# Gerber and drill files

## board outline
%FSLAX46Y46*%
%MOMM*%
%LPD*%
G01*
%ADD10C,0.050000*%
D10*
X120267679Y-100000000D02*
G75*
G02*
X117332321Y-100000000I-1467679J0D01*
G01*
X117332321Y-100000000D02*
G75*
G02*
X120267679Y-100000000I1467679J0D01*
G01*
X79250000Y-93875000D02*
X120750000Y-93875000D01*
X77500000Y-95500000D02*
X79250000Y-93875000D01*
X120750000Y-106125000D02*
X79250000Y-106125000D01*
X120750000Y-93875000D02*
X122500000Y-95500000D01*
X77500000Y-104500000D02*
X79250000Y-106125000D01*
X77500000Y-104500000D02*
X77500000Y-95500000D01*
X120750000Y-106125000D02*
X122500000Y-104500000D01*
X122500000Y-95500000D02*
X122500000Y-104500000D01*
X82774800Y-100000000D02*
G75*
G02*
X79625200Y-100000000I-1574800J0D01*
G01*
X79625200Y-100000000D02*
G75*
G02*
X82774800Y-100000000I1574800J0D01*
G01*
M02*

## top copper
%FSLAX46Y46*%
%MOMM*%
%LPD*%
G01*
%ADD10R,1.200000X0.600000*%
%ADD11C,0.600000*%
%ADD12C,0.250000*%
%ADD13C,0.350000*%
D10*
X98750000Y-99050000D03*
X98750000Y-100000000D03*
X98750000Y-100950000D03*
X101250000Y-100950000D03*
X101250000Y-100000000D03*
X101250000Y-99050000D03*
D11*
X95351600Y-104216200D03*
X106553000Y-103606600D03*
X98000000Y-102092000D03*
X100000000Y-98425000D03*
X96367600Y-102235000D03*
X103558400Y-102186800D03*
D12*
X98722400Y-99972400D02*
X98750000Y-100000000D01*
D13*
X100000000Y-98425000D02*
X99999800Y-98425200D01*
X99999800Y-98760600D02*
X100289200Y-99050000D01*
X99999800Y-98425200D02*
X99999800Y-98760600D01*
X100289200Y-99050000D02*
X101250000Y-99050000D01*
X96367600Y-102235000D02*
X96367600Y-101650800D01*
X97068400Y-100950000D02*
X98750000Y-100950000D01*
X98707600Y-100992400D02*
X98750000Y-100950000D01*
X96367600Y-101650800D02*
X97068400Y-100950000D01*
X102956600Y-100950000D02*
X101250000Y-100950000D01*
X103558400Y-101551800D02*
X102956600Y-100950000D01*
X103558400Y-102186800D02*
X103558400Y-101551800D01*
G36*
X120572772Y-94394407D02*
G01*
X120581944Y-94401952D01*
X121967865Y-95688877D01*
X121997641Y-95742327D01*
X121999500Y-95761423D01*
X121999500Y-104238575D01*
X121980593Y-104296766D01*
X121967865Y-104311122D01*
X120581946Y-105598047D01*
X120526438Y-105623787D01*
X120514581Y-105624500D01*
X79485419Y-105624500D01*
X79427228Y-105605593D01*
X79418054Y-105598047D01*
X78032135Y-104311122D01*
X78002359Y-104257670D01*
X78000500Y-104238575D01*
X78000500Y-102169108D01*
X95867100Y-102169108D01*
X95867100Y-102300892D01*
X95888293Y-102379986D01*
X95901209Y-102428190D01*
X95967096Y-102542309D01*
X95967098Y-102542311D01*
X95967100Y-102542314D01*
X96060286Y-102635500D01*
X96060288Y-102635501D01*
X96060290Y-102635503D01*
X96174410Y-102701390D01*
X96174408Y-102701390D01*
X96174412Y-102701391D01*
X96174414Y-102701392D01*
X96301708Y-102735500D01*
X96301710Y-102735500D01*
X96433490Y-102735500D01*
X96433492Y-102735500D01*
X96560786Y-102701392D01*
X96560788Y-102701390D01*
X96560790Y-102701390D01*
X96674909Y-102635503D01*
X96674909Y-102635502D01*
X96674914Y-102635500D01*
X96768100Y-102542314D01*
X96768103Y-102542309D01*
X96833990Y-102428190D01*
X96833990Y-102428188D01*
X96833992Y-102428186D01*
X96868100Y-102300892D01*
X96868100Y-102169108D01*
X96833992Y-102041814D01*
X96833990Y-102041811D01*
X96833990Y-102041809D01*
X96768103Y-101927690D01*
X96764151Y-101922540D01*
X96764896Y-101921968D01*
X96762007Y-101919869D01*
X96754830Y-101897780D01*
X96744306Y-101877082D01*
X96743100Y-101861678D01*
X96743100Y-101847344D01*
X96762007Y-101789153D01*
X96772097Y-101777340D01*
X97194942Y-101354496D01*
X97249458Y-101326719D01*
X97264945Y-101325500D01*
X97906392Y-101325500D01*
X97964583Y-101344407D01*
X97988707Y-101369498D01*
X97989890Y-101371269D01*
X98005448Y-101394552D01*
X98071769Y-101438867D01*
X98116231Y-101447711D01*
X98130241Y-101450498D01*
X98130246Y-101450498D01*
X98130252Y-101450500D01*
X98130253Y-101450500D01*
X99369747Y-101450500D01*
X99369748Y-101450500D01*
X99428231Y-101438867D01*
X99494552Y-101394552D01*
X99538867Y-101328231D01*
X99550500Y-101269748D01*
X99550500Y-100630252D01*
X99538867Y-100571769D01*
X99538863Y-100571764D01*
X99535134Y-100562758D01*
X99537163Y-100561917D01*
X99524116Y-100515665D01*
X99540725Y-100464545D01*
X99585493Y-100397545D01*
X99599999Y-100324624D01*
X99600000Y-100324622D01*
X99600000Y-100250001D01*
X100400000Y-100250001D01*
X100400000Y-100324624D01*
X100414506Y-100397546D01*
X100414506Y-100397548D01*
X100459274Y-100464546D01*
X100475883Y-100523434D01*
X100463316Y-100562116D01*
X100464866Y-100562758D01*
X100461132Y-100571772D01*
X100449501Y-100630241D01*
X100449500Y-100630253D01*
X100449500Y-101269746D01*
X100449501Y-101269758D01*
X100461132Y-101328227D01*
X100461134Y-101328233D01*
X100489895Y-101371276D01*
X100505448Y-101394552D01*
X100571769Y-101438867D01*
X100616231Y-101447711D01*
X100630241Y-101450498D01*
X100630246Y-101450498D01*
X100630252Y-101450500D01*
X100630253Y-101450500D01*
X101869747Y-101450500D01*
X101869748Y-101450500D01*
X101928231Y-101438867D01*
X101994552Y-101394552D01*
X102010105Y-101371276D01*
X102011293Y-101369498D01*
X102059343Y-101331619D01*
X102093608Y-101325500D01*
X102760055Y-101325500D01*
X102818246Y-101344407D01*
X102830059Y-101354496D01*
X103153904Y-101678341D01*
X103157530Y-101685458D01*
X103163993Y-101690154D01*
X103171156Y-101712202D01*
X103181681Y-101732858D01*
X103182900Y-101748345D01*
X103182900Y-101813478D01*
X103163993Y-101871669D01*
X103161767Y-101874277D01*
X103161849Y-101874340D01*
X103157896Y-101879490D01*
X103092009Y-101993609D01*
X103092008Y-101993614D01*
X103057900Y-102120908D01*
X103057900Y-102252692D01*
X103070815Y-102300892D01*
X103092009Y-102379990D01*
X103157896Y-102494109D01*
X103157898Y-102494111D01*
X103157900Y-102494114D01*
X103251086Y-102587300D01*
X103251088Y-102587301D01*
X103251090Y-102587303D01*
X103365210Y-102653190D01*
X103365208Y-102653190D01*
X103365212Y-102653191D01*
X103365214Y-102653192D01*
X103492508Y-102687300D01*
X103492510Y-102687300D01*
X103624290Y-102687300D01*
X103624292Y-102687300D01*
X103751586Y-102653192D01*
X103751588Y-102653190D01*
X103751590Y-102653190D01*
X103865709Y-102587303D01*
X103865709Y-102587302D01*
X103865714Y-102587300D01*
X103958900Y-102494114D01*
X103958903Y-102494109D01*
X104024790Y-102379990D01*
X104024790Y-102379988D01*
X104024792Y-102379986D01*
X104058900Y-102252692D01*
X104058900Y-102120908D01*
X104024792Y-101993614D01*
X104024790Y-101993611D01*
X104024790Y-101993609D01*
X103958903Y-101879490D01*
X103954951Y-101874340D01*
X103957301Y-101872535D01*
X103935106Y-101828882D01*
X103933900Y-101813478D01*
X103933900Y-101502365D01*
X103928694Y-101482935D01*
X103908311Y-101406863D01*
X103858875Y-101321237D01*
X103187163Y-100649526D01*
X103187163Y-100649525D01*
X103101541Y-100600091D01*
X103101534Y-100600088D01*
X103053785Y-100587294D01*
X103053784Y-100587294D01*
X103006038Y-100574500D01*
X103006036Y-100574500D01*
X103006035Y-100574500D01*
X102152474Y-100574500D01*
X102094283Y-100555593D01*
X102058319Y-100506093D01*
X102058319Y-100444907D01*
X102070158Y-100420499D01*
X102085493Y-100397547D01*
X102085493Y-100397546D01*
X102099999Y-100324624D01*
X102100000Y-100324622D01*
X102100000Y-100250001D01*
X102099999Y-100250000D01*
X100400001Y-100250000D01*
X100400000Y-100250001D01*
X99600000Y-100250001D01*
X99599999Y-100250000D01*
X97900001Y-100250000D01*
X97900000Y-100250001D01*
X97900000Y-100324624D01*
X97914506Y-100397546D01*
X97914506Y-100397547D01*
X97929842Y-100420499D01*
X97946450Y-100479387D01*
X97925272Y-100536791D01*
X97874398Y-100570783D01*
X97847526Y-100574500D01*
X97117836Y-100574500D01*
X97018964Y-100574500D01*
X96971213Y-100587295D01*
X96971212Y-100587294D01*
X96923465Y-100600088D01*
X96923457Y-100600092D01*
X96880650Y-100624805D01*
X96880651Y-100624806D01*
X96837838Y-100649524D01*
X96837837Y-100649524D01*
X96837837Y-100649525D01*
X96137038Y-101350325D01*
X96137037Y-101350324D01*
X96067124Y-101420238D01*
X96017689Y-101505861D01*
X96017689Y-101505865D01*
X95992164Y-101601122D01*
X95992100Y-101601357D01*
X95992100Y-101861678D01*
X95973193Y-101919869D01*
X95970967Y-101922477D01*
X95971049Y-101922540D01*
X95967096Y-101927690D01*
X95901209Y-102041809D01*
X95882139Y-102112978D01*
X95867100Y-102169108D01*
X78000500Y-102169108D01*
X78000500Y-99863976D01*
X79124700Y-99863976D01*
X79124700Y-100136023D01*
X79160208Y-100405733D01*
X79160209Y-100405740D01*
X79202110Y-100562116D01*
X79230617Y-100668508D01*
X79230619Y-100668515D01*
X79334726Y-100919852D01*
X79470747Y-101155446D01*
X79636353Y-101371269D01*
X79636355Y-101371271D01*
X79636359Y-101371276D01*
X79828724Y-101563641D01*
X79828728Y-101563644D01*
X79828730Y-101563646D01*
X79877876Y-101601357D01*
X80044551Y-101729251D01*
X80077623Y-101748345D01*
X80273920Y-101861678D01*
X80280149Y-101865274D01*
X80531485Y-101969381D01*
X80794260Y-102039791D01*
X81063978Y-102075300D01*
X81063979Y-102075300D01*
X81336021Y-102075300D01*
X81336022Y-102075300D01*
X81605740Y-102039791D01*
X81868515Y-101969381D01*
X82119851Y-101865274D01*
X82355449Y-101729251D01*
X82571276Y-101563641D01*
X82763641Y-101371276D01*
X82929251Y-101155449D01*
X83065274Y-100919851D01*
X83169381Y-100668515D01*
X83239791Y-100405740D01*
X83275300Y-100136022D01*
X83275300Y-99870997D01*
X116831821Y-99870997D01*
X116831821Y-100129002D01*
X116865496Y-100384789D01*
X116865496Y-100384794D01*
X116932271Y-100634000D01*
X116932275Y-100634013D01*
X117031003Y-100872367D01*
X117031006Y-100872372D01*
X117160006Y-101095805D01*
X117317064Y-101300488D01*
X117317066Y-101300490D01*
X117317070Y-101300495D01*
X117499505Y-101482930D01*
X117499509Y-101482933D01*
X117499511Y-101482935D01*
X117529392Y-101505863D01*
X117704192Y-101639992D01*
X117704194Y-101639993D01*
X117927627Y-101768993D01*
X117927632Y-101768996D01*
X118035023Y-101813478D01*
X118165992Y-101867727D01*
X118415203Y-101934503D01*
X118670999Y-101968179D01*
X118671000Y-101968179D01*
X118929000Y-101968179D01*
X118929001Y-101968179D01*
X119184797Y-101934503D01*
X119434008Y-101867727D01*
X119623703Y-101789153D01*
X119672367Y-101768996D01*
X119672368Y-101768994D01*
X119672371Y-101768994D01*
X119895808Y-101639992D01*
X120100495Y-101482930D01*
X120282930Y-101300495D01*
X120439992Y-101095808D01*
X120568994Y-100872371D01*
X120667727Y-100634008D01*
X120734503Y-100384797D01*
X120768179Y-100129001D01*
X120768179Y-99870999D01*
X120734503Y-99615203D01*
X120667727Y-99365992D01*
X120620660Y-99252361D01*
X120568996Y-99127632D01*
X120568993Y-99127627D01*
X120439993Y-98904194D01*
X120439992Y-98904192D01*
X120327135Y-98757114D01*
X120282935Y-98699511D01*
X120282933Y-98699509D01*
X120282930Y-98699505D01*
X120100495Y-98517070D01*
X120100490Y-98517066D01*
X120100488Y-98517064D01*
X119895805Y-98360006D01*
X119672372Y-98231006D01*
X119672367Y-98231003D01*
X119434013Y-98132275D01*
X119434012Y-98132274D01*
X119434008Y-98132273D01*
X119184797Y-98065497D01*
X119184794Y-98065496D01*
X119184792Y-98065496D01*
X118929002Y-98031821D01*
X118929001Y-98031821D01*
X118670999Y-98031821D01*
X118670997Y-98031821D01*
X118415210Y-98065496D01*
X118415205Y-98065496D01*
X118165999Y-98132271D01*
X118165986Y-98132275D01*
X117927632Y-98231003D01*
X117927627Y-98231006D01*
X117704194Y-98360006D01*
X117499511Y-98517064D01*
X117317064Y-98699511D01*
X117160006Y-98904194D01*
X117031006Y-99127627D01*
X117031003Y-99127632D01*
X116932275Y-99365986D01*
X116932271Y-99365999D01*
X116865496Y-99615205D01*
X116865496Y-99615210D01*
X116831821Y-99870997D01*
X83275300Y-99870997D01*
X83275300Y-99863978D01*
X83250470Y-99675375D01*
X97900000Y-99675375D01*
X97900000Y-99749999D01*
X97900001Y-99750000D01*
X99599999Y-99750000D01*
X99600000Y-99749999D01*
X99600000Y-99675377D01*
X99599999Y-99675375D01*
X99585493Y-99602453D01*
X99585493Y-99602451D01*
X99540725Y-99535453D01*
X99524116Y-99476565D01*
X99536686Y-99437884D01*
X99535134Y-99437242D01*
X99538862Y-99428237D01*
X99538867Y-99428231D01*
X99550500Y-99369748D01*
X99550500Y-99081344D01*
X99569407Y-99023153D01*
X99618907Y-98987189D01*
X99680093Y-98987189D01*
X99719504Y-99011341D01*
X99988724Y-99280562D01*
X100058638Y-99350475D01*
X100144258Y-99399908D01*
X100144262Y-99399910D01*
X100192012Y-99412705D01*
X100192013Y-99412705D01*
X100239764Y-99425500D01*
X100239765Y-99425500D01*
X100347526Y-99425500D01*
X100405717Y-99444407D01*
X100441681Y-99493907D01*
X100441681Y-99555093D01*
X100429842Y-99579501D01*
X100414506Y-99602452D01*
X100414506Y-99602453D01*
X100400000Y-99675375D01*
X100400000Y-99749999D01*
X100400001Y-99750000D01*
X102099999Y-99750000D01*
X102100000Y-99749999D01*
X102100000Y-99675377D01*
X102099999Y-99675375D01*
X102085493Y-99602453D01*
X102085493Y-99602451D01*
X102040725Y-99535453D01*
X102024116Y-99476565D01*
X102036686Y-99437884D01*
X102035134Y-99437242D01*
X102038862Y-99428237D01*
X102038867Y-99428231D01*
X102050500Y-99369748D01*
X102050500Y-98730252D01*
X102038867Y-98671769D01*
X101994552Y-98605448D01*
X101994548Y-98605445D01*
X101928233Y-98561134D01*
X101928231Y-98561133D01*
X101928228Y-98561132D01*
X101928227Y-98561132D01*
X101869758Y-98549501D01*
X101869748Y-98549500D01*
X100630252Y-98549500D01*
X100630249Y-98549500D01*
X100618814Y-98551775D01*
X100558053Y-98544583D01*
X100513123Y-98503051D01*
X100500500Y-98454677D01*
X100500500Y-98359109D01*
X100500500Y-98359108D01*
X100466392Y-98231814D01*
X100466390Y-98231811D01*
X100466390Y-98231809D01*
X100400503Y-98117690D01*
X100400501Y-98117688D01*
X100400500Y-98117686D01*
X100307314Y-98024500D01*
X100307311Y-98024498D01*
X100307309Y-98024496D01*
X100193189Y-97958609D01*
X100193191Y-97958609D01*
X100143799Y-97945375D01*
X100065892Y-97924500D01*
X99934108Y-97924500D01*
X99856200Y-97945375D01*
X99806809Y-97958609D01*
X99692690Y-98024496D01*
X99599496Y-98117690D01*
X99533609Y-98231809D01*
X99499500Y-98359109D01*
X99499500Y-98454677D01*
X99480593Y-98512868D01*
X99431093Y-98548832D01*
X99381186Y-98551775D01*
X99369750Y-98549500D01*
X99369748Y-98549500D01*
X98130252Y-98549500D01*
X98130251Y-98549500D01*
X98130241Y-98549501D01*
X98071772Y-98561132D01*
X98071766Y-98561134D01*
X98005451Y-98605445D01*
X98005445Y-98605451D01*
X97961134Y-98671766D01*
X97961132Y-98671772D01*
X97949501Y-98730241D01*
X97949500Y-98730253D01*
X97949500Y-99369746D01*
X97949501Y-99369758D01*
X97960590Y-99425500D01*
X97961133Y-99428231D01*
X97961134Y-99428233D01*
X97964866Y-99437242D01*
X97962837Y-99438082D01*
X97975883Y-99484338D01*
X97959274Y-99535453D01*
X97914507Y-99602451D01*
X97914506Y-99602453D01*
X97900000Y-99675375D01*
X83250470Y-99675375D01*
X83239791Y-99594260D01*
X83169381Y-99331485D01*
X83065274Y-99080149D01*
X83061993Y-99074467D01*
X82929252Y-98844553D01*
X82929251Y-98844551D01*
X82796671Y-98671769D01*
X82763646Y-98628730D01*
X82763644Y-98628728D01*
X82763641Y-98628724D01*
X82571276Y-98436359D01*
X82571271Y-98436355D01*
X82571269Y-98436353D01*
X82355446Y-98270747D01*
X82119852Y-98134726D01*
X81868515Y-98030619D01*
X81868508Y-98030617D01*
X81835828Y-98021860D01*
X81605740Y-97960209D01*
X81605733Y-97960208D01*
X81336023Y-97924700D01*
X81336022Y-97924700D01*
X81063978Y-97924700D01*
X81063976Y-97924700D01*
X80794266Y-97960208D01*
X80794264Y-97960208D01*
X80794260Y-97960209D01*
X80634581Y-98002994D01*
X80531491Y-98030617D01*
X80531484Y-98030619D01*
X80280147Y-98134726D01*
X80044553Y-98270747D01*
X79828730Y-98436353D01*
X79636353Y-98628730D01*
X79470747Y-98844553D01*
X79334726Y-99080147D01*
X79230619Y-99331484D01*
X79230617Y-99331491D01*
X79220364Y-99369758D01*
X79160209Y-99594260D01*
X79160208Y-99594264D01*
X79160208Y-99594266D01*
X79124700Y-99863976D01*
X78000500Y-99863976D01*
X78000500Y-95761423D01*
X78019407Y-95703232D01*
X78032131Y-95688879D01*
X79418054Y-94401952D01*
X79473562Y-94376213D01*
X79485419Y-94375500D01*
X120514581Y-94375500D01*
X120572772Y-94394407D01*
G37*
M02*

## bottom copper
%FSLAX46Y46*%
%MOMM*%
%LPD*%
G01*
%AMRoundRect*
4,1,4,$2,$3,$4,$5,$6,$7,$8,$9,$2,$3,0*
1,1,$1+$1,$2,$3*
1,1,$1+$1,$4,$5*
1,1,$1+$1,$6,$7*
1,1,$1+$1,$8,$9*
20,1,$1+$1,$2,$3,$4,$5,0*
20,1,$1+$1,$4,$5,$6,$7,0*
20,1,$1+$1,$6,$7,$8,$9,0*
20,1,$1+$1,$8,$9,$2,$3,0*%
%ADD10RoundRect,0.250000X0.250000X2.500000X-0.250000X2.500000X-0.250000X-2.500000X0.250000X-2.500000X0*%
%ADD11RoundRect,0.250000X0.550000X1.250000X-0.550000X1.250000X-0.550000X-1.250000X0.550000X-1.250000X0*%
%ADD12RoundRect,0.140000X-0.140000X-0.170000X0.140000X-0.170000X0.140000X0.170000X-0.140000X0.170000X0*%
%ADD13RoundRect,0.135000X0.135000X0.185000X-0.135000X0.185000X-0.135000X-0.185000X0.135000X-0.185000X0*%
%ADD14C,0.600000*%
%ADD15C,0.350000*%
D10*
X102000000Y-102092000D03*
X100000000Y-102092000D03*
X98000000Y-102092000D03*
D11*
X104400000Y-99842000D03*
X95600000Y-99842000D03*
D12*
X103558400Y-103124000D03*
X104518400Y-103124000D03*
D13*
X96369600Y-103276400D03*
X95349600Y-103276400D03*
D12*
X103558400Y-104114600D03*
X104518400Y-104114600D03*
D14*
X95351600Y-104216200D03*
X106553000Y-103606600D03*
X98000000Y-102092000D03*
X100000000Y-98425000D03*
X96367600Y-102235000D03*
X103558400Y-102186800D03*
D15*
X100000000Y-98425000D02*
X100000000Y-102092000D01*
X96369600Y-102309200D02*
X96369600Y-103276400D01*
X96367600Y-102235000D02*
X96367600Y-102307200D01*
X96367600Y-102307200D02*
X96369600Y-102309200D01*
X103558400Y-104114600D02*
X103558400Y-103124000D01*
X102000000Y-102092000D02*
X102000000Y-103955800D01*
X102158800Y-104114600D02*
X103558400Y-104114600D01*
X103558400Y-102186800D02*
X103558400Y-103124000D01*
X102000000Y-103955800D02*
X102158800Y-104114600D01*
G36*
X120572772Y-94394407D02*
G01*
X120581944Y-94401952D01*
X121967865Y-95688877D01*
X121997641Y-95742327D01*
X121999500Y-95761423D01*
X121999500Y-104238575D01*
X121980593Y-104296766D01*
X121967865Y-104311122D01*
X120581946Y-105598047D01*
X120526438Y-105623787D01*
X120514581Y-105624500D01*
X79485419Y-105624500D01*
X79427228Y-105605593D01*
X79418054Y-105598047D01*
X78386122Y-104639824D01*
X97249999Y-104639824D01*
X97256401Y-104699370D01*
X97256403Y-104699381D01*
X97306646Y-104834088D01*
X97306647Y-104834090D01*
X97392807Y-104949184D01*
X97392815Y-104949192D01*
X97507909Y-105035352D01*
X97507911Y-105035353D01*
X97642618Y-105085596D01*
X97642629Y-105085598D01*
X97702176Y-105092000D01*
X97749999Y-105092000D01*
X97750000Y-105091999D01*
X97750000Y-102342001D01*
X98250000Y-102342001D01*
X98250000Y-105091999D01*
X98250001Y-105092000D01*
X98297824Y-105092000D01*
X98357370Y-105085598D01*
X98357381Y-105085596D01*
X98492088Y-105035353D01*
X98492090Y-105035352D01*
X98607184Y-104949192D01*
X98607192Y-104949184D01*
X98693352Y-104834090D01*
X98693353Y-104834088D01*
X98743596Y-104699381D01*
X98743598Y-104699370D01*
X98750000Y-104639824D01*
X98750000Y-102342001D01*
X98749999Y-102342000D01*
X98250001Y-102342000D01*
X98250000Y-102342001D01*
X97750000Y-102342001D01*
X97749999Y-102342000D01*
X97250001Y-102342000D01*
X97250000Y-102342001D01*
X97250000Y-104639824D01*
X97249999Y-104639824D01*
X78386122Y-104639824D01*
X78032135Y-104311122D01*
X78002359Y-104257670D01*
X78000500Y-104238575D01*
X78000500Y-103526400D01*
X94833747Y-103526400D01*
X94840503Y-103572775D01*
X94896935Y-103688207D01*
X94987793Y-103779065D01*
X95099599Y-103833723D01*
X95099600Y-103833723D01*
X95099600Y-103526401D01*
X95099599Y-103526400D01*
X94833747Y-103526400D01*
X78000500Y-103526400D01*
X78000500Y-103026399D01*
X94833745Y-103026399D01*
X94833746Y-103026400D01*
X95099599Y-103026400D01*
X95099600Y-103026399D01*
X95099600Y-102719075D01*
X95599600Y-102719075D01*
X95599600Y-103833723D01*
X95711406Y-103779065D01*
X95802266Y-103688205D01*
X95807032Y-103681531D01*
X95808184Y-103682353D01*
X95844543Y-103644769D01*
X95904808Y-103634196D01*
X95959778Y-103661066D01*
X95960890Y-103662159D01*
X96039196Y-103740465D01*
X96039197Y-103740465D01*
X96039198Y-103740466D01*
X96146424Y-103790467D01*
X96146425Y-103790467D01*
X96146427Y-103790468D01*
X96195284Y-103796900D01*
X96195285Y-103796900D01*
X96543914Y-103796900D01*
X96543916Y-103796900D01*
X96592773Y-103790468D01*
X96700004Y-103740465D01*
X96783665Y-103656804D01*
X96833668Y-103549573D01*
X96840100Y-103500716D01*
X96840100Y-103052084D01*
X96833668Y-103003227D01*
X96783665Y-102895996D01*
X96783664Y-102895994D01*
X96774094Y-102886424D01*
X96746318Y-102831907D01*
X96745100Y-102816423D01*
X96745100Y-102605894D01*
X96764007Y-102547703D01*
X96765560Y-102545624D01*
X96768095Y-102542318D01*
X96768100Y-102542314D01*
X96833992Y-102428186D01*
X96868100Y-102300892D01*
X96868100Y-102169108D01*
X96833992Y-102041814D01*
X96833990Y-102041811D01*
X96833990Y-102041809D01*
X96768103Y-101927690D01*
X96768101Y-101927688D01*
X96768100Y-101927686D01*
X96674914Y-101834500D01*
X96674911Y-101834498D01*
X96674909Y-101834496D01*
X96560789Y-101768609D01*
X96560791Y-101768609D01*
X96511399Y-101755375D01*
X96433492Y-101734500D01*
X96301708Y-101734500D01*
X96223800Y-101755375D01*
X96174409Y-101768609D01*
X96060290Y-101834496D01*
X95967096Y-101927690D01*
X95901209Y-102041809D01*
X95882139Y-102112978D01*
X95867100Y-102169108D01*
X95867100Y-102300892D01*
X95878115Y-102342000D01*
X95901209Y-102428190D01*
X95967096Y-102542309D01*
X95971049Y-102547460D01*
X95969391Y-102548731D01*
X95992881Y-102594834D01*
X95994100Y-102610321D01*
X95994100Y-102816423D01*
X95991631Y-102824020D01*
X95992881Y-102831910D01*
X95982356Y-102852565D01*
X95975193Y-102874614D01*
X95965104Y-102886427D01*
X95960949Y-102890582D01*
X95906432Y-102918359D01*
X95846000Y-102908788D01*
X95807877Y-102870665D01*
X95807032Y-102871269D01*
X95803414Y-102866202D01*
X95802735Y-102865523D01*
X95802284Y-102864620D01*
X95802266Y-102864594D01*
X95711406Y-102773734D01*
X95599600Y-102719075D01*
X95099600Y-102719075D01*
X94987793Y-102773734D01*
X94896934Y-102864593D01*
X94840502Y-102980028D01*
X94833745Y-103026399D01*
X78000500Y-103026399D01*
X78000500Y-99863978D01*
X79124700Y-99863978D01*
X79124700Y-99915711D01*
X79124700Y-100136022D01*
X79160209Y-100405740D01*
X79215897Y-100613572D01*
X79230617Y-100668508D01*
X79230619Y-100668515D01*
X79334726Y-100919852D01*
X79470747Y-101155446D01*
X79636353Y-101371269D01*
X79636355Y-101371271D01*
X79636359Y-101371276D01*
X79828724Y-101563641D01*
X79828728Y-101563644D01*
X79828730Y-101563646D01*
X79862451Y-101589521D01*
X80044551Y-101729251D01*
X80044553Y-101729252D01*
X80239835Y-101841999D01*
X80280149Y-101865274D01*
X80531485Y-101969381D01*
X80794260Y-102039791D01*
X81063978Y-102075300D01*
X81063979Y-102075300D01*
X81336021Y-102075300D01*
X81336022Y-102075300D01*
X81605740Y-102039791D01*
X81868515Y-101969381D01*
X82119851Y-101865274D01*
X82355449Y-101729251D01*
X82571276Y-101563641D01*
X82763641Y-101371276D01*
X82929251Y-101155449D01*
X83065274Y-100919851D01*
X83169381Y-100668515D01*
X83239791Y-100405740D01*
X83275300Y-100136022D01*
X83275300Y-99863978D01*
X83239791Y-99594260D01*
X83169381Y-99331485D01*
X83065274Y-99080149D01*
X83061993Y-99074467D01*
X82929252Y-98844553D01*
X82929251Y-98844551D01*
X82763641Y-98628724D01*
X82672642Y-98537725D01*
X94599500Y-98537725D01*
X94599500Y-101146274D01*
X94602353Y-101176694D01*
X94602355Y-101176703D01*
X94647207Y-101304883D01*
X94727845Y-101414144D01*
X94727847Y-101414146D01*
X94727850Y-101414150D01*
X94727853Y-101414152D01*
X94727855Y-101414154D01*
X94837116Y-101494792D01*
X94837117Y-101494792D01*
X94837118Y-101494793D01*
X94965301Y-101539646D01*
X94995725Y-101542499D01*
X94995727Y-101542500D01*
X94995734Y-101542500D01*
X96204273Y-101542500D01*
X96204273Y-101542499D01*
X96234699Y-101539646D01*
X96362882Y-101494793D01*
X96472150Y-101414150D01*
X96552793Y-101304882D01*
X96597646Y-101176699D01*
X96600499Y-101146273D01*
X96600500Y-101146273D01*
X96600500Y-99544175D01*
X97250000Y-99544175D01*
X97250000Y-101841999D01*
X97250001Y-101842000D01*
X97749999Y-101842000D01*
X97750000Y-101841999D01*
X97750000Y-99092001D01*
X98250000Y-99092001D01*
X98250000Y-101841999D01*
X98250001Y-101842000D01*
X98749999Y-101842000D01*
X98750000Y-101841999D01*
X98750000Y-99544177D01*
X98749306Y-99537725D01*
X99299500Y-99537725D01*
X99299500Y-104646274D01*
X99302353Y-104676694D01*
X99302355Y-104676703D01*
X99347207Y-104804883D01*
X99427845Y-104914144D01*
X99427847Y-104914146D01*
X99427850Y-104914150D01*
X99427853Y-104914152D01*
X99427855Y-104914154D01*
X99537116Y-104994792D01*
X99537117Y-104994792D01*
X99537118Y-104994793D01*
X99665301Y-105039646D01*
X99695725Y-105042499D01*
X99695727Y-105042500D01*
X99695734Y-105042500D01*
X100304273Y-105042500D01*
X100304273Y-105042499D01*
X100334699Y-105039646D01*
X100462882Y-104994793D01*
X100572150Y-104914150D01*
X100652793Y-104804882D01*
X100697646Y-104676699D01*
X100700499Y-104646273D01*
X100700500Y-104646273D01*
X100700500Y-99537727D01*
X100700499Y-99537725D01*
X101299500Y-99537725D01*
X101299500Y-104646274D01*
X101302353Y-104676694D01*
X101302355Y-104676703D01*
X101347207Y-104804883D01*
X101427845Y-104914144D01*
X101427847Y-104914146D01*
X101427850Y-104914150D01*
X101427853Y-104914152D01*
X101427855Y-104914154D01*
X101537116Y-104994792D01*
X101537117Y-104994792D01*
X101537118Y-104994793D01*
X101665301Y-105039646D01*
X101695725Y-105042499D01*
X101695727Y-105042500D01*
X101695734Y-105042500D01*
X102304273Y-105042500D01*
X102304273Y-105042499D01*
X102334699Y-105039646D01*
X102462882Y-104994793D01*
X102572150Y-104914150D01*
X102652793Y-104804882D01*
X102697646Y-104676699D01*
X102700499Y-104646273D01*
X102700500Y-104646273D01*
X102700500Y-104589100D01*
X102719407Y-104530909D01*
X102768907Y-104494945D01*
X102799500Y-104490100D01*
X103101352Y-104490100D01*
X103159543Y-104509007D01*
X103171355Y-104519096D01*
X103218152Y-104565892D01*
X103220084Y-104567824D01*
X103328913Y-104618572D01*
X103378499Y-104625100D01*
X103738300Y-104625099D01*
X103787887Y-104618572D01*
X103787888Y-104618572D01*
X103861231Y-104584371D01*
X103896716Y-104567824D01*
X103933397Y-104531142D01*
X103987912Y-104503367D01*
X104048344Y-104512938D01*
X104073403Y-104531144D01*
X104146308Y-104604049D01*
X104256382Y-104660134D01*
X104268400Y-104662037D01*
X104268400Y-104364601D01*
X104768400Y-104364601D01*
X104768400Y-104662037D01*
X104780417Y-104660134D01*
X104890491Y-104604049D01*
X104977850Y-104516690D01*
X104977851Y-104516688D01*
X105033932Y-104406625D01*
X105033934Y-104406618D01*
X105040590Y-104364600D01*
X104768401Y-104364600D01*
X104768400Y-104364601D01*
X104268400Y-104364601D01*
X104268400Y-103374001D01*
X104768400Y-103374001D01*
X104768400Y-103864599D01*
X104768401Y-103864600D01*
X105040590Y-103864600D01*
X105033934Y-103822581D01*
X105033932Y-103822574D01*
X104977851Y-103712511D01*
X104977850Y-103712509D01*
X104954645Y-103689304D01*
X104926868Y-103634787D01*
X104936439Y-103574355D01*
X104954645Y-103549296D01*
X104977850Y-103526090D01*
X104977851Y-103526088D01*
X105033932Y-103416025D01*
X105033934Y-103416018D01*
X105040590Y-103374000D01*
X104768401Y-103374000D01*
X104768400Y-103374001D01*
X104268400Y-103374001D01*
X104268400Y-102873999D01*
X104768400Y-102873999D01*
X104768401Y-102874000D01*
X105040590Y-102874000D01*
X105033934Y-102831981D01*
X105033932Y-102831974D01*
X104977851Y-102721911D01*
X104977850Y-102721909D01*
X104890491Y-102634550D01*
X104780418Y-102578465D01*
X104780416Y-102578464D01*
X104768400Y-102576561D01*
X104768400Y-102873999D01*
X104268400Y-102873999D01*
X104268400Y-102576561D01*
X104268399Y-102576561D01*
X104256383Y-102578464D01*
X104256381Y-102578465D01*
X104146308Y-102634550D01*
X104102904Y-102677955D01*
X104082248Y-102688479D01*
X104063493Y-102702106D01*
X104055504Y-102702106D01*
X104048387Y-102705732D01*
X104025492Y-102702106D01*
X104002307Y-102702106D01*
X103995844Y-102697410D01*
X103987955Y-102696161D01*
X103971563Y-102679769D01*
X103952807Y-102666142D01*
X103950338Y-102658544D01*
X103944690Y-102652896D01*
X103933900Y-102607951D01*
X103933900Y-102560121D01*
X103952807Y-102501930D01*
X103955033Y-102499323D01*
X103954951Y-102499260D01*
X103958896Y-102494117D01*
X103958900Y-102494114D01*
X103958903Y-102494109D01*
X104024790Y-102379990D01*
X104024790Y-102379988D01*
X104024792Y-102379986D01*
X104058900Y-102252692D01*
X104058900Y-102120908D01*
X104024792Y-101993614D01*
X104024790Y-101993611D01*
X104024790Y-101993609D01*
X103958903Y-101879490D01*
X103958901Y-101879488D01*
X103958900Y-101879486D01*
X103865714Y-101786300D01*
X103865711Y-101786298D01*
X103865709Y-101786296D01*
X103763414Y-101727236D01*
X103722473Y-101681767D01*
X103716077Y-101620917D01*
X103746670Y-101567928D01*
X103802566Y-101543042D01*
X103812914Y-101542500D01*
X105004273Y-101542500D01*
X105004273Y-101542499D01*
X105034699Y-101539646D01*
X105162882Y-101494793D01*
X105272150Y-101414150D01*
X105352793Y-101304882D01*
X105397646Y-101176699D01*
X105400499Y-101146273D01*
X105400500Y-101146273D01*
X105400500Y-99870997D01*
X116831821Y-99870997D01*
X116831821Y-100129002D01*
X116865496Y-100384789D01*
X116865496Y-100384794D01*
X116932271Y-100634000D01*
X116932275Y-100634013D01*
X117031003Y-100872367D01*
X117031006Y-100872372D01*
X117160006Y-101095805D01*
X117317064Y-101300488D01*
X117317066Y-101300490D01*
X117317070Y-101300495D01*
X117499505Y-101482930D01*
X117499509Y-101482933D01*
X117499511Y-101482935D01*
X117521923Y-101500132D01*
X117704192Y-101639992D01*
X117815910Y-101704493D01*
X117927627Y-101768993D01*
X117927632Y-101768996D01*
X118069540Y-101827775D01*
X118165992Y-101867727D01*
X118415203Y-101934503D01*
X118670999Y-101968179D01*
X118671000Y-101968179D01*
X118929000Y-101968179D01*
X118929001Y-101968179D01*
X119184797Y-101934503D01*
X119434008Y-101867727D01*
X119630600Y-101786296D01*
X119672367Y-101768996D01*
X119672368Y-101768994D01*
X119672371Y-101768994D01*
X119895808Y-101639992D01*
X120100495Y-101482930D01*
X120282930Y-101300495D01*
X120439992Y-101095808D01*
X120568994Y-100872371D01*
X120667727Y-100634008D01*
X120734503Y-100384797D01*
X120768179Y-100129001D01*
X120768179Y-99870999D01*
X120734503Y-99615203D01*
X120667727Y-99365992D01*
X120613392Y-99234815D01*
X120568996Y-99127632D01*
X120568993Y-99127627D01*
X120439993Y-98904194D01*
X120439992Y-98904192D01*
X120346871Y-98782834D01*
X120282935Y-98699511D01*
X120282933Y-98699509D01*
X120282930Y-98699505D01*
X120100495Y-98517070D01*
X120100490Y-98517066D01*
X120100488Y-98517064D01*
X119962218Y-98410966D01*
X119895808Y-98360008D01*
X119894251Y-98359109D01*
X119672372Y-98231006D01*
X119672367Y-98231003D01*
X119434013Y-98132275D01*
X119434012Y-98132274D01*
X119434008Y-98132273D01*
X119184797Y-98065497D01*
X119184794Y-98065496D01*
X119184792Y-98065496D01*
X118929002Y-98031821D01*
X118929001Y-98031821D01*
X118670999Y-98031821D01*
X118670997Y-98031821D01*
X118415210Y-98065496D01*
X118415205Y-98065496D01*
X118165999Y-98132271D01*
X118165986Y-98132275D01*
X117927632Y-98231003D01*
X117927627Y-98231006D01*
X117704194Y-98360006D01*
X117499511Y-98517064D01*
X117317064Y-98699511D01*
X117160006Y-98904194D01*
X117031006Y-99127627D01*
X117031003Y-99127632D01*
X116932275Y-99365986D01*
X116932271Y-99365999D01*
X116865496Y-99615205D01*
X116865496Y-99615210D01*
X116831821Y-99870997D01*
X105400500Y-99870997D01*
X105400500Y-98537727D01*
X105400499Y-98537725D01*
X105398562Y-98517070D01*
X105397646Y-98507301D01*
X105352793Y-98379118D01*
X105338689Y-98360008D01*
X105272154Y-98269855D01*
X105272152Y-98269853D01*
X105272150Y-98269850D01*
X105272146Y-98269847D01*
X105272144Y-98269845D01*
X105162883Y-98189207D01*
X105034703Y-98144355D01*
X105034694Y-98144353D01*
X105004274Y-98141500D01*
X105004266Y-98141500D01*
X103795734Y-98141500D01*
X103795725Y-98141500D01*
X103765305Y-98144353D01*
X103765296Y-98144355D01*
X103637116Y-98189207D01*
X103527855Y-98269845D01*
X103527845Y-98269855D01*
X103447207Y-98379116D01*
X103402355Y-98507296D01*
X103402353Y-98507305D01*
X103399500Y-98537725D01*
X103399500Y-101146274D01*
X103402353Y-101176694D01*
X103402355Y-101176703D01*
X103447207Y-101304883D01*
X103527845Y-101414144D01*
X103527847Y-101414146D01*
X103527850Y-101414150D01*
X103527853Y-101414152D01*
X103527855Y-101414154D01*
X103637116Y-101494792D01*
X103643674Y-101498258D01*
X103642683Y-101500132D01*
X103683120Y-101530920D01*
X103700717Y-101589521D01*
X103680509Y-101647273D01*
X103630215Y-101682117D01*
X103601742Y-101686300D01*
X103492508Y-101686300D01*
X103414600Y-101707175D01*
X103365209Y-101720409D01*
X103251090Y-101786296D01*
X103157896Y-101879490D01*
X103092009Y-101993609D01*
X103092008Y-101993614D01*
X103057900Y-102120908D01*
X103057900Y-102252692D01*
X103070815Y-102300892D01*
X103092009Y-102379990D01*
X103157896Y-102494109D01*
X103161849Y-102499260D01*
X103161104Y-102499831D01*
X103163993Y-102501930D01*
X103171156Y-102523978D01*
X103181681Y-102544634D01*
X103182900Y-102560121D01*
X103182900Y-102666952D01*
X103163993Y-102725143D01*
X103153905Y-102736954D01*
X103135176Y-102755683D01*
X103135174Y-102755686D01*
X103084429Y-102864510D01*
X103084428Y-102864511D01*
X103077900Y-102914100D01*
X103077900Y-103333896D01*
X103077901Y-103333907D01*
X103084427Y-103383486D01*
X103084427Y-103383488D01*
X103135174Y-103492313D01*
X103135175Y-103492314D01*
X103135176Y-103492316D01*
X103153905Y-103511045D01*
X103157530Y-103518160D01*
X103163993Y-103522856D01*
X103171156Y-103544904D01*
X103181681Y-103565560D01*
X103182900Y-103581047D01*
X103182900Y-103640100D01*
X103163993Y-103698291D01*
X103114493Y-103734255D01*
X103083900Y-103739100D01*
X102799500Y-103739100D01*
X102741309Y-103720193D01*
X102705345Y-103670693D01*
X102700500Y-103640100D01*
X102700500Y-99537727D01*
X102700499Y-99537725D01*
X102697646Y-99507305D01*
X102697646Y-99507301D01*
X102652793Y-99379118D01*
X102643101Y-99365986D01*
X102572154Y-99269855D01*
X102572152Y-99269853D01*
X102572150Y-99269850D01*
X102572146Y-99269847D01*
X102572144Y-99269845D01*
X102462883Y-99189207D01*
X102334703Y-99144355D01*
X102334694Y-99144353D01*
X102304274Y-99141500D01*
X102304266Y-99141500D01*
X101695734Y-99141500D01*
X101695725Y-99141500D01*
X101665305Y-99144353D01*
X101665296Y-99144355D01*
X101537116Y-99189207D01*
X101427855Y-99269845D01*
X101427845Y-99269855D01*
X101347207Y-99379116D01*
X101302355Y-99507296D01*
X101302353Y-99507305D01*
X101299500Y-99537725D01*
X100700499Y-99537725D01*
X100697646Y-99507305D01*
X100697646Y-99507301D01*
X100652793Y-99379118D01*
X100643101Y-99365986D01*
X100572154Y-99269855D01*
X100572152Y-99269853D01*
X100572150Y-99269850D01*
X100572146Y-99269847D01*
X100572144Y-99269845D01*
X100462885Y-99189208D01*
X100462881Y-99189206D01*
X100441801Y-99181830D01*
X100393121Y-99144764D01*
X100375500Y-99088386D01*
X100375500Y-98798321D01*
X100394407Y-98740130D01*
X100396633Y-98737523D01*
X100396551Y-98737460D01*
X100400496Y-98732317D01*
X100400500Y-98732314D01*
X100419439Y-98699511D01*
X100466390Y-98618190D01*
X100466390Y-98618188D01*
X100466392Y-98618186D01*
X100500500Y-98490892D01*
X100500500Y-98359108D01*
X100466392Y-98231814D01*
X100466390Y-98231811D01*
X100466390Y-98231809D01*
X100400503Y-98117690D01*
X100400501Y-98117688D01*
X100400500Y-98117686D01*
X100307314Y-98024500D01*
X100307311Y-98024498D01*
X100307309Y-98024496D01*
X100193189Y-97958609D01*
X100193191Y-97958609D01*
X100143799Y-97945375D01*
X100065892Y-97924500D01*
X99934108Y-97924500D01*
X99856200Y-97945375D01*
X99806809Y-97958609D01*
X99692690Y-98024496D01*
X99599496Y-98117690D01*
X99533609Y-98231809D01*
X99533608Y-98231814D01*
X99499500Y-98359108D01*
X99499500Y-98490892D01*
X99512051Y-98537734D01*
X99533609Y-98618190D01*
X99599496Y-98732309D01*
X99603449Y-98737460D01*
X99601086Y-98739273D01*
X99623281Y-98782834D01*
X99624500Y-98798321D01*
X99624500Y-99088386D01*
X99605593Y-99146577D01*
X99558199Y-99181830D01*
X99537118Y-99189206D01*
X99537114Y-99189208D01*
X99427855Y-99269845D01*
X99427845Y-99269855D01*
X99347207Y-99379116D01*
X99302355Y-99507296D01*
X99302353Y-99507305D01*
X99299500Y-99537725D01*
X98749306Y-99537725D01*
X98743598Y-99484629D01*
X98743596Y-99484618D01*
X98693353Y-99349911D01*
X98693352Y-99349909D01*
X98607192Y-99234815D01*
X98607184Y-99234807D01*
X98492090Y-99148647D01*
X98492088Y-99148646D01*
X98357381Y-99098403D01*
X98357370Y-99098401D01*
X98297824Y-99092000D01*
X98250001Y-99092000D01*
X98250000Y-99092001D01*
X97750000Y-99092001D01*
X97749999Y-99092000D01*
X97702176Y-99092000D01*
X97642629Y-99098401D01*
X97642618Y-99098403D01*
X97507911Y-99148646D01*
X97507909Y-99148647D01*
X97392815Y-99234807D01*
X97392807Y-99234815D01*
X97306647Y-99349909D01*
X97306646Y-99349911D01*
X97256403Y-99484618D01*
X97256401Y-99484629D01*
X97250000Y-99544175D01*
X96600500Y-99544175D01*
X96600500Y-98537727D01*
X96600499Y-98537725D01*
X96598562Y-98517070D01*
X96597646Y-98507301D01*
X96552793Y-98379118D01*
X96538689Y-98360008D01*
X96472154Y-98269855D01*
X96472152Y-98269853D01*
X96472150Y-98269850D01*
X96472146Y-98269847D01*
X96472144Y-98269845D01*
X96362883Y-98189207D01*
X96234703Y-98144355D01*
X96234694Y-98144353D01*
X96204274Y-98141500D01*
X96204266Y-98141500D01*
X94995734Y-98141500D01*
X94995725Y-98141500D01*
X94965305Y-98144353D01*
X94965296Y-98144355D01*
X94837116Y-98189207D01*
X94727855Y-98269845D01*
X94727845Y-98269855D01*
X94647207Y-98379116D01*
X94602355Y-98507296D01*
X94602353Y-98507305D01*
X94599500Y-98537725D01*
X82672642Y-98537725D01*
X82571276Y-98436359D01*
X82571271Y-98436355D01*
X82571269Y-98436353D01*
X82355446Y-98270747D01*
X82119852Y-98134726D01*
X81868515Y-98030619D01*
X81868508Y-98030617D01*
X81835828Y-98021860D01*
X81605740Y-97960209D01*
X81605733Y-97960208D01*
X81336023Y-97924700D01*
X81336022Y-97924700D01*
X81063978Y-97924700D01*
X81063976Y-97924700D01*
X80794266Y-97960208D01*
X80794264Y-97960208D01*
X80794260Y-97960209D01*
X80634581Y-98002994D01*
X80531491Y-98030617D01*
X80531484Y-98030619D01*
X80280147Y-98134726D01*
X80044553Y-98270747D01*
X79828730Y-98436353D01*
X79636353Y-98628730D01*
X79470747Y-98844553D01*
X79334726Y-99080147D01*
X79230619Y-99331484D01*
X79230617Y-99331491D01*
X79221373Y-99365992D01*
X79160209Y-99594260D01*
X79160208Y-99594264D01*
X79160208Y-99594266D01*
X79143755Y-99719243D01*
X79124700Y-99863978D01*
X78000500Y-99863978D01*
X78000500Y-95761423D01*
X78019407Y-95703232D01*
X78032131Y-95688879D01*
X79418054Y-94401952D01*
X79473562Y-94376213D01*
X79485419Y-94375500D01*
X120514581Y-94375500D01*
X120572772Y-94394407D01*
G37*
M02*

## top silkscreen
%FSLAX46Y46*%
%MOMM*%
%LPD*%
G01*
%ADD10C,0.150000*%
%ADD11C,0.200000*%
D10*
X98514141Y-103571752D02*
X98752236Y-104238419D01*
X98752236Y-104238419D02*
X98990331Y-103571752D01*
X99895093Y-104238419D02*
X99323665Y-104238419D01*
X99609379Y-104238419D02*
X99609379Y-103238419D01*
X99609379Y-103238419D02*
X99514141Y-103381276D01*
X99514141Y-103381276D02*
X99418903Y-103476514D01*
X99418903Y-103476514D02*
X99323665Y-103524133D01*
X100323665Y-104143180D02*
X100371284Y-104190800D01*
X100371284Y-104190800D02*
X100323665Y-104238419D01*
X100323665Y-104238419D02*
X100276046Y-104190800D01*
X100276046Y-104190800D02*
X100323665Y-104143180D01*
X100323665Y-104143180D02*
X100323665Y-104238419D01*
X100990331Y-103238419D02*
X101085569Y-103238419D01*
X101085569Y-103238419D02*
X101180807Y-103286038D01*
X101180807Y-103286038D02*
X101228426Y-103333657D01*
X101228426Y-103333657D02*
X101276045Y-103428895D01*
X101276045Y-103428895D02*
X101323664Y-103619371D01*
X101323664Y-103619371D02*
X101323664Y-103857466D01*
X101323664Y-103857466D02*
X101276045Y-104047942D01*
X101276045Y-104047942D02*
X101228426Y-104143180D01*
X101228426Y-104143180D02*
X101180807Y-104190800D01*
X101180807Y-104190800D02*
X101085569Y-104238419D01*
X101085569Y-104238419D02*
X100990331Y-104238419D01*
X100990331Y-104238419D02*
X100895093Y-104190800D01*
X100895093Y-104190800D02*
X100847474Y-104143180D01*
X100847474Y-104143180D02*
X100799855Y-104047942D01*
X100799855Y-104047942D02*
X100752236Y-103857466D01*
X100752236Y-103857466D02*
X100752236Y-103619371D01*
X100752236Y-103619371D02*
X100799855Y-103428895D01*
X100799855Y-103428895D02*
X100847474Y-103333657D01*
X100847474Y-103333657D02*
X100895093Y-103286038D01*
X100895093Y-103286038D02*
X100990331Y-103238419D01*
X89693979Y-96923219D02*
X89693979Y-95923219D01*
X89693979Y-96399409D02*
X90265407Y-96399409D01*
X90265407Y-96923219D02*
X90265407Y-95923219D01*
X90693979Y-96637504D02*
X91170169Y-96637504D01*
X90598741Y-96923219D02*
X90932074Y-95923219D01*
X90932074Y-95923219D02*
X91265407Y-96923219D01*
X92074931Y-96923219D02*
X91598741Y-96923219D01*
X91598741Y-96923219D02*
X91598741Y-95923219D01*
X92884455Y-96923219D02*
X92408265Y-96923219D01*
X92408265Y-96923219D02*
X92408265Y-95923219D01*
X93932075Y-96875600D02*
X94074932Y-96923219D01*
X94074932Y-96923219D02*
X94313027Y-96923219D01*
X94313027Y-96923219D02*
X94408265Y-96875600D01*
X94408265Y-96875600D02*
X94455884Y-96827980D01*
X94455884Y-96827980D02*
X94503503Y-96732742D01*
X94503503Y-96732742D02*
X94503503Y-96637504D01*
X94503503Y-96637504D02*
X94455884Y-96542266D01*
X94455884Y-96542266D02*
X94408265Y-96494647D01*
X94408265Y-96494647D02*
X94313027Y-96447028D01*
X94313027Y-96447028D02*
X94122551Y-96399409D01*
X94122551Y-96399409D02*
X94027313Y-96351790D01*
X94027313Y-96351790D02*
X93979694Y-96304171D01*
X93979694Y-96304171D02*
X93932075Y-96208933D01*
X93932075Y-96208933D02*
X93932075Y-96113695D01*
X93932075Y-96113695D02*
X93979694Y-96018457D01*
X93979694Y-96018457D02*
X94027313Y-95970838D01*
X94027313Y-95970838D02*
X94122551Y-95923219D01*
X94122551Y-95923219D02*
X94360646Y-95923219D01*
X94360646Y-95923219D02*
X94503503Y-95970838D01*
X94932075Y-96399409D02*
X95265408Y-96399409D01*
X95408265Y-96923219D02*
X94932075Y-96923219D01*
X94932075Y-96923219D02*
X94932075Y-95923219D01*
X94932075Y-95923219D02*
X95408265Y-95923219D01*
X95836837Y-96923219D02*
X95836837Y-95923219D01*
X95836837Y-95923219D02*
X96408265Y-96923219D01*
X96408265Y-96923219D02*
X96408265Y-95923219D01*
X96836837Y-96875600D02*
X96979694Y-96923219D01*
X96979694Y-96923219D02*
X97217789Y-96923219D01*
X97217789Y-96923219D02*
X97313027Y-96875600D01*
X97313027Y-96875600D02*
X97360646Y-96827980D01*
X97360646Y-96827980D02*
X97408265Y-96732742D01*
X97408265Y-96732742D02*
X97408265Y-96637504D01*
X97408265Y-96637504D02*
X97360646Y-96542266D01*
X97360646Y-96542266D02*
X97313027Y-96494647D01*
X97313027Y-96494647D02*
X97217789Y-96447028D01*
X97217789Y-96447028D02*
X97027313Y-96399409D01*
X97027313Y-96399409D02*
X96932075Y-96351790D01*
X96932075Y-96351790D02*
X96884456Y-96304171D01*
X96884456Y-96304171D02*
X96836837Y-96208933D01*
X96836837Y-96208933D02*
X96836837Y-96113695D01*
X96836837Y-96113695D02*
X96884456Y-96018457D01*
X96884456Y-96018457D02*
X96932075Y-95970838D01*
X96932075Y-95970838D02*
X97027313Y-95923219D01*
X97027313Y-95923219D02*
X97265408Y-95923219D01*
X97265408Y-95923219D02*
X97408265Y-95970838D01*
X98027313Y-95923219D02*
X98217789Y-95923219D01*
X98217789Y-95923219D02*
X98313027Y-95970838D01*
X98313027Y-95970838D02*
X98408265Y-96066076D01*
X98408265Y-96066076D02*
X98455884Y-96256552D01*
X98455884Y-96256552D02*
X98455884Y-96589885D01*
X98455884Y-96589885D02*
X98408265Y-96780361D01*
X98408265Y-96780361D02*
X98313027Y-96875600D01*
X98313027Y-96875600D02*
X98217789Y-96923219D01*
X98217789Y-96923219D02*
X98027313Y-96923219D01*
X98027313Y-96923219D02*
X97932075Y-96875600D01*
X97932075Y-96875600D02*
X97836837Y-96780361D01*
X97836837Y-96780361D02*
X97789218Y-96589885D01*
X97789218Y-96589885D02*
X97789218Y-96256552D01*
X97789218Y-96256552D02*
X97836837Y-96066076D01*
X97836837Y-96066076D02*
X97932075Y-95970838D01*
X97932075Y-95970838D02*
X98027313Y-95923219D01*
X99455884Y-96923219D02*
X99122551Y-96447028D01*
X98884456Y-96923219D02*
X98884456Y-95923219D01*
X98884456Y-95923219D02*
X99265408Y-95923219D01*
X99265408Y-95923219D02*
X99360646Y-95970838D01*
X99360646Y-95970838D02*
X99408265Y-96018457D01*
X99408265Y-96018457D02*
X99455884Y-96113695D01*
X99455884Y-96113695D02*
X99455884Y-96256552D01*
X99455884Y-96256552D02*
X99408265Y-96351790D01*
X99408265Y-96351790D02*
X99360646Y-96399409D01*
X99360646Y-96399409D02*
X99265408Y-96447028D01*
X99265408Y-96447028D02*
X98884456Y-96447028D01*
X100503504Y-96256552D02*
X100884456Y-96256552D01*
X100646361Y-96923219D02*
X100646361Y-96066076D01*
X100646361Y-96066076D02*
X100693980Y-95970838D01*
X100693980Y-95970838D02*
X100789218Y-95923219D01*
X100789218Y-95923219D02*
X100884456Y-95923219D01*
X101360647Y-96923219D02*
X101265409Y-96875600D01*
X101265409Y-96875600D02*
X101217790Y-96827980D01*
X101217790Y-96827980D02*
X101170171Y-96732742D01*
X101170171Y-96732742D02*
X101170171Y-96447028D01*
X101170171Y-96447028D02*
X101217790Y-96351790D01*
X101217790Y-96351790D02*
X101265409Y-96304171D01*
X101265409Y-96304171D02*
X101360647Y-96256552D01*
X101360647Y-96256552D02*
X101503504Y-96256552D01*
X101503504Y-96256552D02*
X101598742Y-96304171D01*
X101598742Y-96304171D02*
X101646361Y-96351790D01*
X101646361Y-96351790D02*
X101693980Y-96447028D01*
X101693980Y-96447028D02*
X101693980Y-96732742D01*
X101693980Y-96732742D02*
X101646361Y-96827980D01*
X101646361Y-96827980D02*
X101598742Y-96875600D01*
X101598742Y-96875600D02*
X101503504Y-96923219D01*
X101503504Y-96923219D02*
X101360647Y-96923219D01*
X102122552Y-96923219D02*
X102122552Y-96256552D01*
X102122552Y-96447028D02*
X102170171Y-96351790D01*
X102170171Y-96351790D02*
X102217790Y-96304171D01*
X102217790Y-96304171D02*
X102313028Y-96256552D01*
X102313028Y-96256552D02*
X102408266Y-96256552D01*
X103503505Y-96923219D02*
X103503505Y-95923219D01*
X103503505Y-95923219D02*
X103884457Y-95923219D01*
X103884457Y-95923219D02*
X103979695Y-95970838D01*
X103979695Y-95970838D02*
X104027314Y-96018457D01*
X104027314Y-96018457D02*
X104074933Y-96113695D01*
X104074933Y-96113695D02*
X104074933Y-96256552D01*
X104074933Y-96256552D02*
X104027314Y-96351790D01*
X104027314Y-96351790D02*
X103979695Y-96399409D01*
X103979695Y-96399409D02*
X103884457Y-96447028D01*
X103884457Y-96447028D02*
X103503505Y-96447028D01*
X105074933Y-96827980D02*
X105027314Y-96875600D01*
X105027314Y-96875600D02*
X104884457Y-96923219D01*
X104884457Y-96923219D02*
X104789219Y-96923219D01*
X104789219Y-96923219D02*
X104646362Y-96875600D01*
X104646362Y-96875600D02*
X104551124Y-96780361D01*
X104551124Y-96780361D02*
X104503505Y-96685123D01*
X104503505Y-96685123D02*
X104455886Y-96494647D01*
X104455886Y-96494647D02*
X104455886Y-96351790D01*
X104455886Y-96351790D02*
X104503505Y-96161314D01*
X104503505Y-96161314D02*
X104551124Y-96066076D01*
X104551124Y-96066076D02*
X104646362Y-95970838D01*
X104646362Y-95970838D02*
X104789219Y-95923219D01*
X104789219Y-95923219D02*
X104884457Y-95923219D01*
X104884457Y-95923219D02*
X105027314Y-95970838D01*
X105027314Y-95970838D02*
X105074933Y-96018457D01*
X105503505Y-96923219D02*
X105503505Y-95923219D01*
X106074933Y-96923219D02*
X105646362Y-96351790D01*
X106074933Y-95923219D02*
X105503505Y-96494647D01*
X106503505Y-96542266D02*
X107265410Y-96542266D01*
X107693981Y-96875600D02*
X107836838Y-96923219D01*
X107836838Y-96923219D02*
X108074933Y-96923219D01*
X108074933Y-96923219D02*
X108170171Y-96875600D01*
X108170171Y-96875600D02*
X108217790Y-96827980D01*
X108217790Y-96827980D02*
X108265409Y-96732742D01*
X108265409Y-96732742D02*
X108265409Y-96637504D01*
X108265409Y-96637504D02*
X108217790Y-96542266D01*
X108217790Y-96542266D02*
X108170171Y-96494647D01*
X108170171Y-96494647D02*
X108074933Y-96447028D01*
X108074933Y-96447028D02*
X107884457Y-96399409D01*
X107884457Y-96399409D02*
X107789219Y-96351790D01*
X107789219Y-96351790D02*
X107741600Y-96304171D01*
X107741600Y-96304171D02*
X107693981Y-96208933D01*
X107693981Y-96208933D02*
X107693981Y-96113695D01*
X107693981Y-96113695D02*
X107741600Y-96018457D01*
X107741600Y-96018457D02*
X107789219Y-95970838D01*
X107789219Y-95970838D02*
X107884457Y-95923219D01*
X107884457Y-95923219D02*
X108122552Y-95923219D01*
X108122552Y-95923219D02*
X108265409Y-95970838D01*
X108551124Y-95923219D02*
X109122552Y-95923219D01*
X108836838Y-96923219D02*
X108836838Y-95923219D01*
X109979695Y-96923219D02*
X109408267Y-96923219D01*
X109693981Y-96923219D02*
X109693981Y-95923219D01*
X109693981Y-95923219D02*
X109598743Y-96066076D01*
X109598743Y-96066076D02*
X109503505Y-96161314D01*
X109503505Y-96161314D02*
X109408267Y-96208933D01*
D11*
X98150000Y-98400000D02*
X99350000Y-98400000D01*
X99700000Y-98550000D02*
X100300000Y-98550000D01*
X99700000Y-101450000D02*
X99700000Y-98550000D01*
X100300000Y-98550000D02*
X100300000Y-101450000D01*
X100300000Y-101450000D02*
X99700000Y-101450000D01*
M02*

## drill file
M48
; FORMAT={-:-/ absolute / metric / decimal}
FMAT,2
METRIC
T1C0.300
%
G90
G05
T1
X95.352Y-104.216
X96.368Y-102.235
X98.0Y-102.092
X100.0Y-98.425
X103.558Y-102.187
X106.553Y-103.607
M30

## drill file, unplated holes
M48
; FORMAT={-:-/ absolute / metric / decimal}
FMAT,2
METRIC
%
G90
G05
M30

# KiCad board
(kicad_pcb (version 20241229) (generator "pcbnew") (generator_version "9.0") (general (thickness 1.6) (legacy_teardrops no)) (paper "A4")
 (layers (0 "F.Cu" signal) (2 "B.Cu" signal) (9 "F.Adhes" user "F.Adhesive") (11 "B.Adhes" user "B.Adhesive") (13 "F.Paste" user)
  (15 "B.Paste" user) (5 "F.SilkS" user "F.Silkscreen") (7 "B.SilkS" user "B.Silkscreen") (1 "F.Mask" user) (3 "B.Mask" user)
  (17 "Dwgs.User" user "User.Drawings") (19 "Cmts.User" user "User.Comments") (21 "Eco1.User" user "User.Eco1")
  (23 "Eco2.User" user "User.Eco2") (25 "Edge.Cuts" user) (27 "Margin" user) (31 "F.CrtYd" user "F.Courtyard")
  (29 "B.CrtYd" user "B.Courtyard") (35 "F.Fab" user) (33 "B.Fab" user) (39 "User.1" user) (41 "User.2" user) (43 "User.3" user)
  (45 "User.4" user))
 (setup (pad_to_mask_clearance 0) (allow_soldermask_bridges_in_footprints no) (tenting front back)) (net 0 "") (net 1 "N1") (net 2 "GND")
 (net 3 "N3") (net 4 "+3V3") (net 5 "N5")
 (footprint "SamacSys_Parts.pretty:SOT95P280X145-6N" (layer "F.Cu") (at 100 100)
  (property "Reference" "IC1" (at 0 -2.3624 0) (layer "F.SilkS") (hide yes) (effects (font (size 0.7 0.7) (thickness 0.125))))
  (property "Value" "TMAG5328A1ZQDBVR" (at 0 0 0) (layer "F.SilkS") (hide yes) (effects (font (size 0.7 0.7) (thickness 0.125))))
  (fp_line (start -1.85 -1.6) (end -0.65 -1.6) (stroke (width 0.2) (type solid)) (layer "F.SilkS"))
  (fp_line (start -0.3 -1.45) (end 0.3 -1.45) (stroke (width 0.2) (type solid)) (layer "F.SilkS"))
  (fp_line (start -0.3 1.45) (end -0.3 -1.45) (stroke (width 0.2) (type solid)) (layer "F.SilkS"))
  (fp_line (start 0.3 -1.45) (end 0.3 1.45) (stroke (width 0.2) (type solid)) (layer "F.SilkS"))
  (fp_line (start 0.3 1.45) (end -0.3 1.45) (stroke (width 0.2) (type solid)) (layer "F.SilkS"))
  (pad "1" smd rect (at -1.25 -0.95 90) (size 0.6 1.2) (layers "F.Cu" "F.Mask" "F.Paste") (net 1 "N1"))
  (pad "2" smd rect (at -1.25 0 90) (size 0.6 1.2) (layers "F.Cu" "F.Mask" "F.Paste") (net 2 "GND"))
  (pad "3" smd rect (at -1.25 0.95 90) (size 0.6 1.2) (layers "F.Cu" "F.Mask" "F.Paste") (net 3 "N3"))
  (pad "4" smd rect (at 1.25 0.95 90) (size 0.6 1.2) (layers "F.Cu" "F.Mask" "F.Paste") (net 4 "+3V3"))
  (pad "5" smd rect (at 1.25 0 90) (size 0.6 1.2) (layers "F.Cu" "F.Mask" "F.Paste") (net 2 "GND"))
  (pad "6" smd rect (at 1.25 -0.95 90) (size 0.6 1.2) (layers "F.Cu" "F.Mask" "F.Paste") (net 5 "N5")))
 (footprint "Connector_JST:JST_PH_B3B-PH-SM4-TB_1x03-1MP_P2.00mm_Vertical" (layer "B.Cu") (at 100 101.592 180)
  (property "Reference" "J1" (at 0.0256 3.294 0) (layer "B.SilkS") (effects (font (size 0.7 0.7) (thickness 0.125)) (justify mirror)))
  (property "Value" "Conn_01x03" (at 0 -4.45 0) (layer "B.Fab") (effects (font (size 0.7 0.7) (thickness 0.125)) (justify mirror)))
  (pad "1" smd roundrect (at -2 -0.5 180) (size 1 5.5) (layers "B.Cu" "B.Mask" "B.Paste") (roundrect_rratio 0.25) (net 4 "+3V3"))
  (pad "2" smd roundrect (at 0 -0.5 180) (size 1 5.5) (layers "B.Cu" "B.Mask" "B.Paste") (roundrect_rratio 0.25) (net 5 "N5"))
  (pad "3" smd roundrect (at 2 -0.5 180) (size 1 5.5) (layers "B.Cu" "B.Mask" "B.Paste") (roundrect_rratio 0.25) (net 2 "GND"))
  (pad "MP" smd roundrect (at -4.4 1.75 180) (size 1.6 3) (layers "B.Cu" "B.Mask" "B.Paste") (roundrect_rratio 0.15625))
  (pad "MP" smd roundrect (at 4.4 1.75 180) (size 1.6 3) (layers "B.Cu" "B.Mask" "B.Paste") (roundrect_rratio 0.15625)))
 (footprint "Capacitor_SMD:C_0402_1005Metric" (layer "B.Cu") (at 104.0384 103.124)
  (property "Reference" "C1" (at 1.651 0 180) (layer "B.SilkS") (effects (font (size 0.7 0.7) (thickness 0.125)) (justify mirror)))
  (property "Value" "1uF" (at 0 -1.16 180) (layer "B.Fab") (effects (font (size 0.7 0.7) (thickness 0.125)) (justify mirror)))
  (pad "1" smd roundrect (at -0.48 0) (size 0.56 0.62) (layers "B.Cu" "B.Mask" "B.Paste") (roundrect_rratio 0.25) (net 4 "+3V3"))
  (pad "2" smd roundrect (at 0.48 0) (size 0.56 0.62) (layers "B.Cu" "B.Mask" "B.Paste") (roundrect_rratio 0.25) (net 2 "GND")))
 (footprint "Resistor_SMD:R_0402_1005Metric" (layer "B.Cu") (at 95.8596 103.2764 180)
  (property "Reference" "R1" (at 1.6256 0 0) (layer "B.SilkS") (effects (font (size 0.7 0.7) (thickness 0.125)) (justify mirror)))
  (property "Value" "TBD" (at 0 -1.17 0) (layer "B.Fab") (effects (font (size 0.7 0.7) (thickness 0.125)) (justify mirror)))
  (pad "1" smd roundrect (at -0.51 0 180) (size 0.54 0.64) (layers "B.Cu" "B.Mask" "B.Paste") (roundrect_rratio 0.25) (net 3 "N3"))
  (pad "2" smd roundrect (at 0.51 0 180) (size 0.54 0.64) (layers "B.Cu" "B.Mask" "B.Paste") (roundrect_rratio 0.25) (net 2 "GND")))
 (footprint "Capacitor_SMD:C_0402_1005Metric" (layer "B.Cu") (at 104.0384 104.1146)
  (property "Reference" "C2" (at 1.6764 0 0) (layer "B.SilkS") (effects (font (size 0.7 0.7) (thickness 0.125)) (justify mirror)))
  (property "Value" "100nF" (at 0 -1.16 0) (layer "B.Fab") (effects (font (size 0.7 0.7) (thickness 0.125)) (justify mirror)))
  (pad "1" smd roundrect (at -0.48 0) (size 0.56 0.62) (layers "B.Cu" "B.Mask" "B.Paste") (roundrect_rratio 0.25) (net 4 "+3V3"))
  (pad "2" smd roundrect (at 0.48 0) (size 0.56 0.62) (layers "B.Cu" "B.Mask" "B.Paste") (roundrect_rratio 0.25) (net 2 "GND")))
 (gr_circle (center 118.8 100) (end 120.267679 100) (stroke (width 0.05) (type solid)) (fill no) (layer "Edge.Cuts"))
 (gr_line (start 79.25 93.875) (end 120.75 93.875) (stroke (width 0.05) (type solid)) (layer "Edge.Cuts"))
 (gr_line (start 77.5 95.5) (end 79.25 93.875) (stroke (width 0.05) (type default)) (layer "Edge.Cuts"))
 (gr_line (start 120.75 106.125) (end 79.25 106.125) (stroke (width 0.05) (type solid)) (layer "Edge.Cuts"))
 (gr_line (start 120.75 93.875) (end 122.5 95.5) (stroke (width 0.05) (type default)) (layer "Edge.Cuts"))
 (gr_line (start 77.5 104.5) (end 79.25 106.125) (stroke (width 0.05) (type default)) (layer "Edge.Cuts"))
 (gr_line (start 77.5 104.5) (end 77.5 95.5) (stroke (width 0.05) (type solid)) (layer "Edge.Cuts"))
 (gr_line (start 120.75 106.125) (end 122.5 104.5) (stroke (width 0.05) (type default)) (layer "Edge.Cuts"))
 (gr_line (start 122.5 95.5) (end 122.5 104.5) (stroke (width 0.05) (type solid)) (layer "Edge.Cuts"))
 (gr_circle (center 81.2 100) (end 82.7748 100) (stroke (width 0.05) (type solid)) (fill no) (layer "Edge.Cuts"))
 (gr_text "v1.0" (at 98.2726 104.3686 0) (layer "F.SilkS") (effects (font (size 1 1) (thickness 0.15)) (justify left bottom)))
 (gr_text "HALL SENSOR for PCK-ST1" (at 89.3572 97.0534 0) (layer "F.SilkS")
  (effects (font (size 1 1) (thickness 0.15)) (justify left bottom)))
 (segment (start 98.7224 99.9724) (end 98.75 100) (width 0.25) (layer "F.Cu") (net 2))
 (via (at 95.3516 104.2162) (size 0.6) (drill 0.3) (layers "F.Cu" "B.Cu") (free yes) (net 2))
 (via (at 106.553 103.6066) (size 0.6) (drill 0.3) (layers "F.Cu" "B.Cu") (free yes) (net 2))
 (via (at 98 102.092) (size 0.6) (drill 0.3) (layers "F.Cu" "B.Cu") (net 2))
 (segment (start 100 98.425) (end 99.9998 98.4252) (width 0.35) (layer "F.Cu") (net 5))
 (segment (start 99.9998 98.7606) (end 100.2892 99.05) (width 0.35) (layer "F.Cu") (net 5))
 (segment (start 99.9998 98.4252) (end 99.9998 98.7606) (width 0.35) (layer "F.Cu") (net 5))
 (segment (start 100.2892 99.05) (end 101.25 99.05) (width 0.35) (layer "F.Cu") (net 5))
 (via (at 100 98.425) (size 0.6) (drill 0.3) (layers "F.Cu" "B.Cu") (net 5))
 (segment (start 100 98.425) (end 100 102.092) (width 0.35) (layer "B.Cu") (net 5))
 (segment (start 96.3676 102.235) (end 96.3676 101.6508) (width 0.35) (layer "F.Cu") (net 3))
 (segment (start 97.0684 100.95) (end 98.75 100.95) (width 0.35) (layer "F.Cu") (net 3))
 (segment (start 98.7076 100.9924) (end 98.75 100.95) (width 0.35) (layer "F.Cu") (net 3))
 (segment (start 96.3676 101.6508) (end 97.0684 100.95) (width 0.35) (layer "F.Cu") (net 3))
 (via (at 96.3676 102.235) (size 0.6) (drill 0.3) (layers "F.Cu" "B.Cu") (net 3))
 (segment (start 96.3696 102.3092) (end 96.3696 103.2764) (width 0.35) (layer "B.Cu") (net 3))
 (segment (start 96.3676 102.235) (end 96.3676 102.3072) (width 0.35) (layer "B.Cu") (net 3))
 (segment (start 96.3676 102.3072) (end 96.3696 102.3092) (width 0.35) (layer "B.Cu") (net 3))
 (segment (start 102.9566 100.95) (end 101.25 100.95) (width 0.35) (layer "F.Cu") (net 4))
 (segment (start 103.5584 101.5518) (end 102.9566 100.95) (width 0.35) (layer "F.Cu") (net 4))
 (segment (start 103.5584 102.1868) (end 103.5584 101.5518) (width 0.35) (layer "F.Cu") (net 4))
 (via (at 103.5584 102.1868) (size 0.6) (drill 0.3) (layers "F.Cu" "B.Cu") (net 4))
 (segment (start 103.5584 104.1146) (end 103.5584 103.124) (width 0.35) (layer "B.Cu") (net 4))
 (segment (start 102 102.092) (end 102 103.9558) (width 0.35) (layer "B.Cu") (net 4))
 (segment (start 102.1588 104.1146) (end 103.5584 104.1146) (width 0.35) (layer "B.Cu") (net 4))
 (segment (start 103.5584 102.1868) (end 103.5584 103.124) (width 0.35) (layer "B.Cu") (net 4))
 (segment (start 102 103.9558) (end 102.1588 104.1146) (width 0.35) (layer "B.Cu") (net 4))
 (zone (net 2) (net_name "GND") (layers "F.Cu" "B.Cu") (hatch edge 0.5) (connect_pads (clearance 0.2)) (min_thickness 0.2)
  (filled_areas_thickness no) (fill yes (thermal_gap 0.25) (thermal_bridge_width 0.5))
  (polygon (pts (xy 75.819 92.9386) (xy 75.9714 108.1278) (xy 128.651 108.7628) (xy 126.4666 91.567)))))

